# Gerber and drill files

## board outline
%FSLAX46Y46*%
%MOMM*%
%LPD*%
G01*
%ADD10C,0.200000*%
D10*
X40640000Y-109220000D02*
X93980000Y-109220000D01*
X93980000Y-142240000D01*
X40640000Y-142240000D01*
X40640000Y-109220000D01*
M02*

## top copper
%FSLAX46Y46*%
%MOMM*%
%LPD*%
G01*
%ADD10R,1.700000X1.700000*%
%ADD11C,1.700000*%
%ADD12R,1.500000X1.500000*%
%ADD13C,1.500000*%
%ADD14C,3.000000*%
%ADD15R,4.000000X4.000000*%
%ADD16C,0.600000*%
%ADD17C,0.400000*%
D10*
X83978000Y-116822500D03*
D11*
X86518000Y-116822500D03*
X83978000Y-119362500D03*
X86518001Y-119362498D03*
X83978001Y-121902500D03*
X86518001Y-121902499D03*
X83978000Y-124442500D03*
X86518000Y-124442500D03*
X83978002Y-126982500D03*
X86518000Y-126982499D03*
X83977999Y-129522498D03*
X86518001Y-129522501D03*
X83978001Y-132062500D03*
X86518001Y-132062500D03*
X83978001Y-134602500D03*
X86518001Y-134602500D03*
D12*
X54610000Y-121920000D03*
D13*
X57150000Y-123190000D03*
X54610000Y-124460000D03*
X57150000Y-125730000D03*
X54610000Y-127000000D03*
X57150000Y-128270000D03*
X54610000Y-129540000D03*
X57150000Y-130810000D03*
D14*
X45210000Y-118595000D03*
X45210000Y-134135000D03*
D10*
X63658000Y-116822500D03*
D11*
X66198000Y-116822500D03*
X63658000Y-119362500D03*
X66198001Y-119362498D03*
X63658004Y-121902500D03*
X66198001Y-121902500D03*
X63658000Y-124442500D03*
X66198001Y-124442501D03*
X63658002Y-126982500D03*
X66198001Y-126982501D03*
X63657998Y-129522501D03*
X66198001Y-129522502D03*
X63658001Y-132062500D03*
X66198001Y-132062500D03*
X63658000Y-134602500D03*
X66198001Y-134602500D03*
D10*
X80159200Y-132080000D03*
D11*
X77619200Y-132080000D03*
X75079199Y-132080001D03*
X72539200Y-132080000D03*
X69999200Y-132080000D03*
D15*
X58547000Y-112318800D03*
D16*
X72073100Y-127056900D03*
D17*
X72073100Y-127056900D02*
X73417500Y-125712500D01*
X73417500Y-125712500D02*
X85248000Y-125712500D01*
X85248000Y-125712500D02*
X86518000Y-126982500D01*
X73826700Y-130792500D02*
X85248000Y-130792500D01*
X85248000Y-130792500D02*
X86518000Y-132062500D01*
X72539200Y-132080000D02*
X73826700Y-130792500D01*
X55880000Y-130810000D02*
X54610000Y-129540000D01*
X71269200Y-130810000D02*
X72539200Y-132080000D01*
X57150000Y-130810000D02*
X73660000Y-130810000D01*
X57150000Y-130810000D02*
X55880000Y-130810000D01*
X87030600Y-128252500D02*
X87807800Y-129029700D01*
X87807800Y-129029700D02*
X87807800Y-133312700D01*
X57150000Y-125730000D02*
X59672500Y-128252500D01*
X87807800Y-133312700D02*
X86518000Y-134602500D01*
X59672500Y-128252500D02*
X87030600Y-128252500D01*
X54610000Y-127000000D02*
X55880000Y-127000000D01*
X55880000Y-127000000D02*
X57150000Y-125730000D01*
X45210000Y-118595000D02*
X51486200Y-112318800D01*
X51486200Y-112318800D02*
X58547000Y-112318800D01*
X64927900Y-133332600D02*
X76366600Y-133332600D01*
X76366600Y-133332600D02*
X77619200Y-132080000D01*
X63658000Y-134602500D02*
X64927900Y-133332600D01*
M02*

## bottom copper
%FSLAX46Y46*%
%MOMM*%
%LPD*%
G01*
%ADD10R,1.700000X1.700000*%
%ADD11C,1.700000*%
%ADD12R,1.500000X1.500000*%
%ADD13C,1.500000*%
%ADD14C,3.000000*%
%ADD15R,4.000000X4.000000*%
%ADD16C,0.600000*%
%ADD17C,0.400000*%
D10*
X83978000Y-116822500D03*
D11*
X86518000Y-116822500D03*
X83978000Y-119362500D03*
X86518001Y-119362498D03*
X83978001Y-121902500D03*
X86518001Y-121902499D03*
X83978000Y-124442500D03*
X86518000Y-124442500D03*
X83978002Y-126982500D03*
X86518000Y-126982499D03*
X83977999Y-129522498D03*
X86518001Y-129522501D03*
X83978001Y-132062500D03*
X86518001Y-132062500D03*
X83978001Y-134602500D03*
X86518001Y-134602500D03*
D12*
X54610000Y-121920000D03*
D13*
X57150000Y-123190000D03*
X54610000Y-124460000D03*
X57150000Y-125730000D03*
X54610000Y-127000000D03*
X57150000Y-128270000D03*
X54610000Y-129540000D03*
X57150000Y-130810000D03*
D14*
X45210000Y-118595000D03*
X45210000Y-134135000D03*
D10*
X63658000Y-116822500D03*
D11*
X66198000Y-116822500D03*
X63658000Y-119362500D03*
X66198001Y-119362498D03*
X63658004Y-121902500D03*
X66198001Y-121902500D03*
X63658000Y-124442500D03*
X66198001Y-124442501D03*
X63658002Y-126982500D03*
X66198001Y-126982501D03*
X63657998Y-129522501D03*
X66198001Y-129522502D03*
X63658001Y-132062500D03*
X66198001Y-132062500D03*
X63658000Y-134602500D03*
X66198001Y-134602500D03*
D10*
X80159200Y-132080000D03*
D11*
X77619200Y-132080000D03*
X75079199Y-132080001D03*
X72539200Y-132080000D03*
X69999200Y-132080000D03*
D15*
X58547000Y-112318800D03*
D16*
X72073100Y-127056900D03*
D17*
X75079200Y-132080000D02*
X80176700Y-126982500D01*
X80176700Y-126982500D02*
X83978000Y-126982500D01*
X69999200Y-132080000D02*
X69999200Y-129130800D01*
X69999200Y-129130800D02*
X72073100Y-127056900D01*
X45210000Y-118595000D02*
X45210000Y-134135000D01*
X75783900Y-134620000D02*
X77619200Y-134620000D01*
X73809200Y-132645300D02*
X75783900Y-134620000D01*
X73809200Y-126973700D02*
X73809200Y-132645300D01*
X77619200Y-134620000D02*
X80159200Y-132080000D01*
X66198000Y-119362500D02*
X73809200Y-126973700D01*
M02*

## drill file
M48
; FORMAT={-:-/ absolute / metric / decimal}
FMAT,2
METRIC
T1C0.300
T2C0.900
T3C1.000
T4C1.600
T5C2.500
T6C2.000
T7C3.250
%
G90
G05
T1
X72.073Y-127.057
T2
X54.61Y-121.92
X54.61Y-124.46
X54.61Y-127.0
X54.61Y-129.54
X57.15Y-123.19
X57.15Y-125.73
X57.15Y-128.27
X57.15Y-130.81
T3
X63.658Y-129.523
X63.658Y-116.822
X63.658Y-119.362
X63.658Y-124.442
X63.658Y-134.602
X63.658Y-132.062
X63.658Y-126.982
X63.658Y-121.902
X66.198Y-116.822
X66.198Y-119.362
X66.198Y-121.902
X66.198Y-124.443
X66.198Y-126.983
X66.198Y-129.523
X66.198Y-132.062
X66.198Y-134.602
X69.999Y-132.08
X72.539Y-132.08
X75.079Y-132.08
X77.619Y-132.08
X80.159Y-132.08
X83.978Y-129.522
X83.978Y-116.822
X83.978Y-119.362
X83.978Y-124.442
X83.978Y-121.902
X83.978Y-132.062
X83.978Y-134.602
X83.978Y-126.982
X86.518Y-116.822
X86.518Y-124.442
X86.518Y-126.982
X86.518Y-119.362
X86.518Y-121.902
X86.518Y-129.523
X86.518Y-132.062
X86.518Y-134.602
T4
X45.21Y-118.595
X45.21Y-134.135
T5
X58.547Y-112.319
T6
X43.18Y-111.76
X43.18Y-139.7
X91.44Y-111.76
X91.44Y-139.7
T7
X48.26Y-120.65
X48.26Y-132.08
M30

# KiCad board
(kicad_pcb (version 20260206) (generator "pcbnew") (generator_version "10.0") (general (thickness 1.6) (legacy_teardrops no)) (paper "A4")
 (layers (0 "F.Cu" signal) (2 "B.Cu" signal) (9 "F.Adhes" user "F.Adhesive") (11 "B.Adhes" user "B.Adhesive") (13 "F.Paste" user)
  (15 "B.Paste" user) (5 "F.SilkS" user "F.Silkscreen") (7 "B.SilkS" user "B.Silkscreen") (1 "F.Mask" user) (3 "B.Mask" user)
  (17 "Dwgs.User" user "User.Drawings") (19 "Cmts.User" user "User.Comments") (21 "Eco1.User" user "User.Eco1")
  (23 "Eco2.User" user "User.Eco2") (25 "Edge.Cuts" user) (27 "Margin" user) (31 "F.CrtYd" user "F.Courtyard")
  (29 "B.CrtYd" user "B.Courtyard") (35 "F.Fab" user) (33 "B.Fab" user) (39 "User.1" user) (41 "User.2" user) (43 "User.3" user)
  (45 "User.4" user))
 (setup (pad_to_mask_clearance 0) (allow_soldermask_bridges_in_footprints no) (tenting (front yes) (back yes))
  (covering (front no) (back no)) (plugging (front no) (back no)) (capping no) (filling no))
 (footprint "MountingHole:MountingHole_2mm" (layer "F.Cu") (at 43.18 139.7 90)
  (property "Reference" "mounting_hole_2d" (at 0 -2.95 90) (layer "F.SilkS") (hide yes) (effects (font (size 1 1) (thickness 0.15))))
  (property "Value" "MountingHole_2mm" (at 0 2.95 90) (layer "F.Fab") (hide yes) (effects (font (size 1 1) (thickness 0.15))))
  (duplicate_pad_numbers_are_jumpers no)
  (pad "" np_thru_hole circle (at 0 0 90) (size 2 2) (drill 2) (layers "*.Cu" "*.Mask")))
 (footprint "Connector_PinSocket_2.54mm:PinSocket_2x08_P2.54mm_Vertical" (layer "F.Cu") (at 86.5688 116.8225)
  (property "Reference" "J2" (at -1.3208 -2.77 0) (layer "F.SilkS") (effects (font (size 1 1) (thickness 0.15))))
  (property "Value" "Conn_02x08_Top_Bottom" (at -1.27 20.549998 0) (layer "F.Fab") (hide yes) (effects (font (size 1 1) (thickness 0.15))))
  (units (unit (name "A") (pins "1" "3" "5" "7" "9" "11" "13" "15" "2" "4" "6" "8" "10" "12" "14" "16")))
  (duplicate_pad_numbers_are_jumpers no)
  (pad "1" thru_hole rect (at -2.5908 0) (size 1.7 1.7) (drill 1) (layers "*.Cu" "*.Mask") (remove_unused_layers no)
   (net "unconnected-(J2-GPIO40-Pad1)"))
  (pad "2" thru_hole circle (at -0.0508 0) (size 1.7 1.7) (drill 1) (layers "*.Cu" "*.Mask") (remove_unused_layers no)
   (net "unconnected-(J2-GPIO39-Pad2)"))
  (pad "3" thru_hole circle (at -2.5908 2.54) (size 1.7 1.7) (drill 1) (layers "*.Cu" "*.Mask") (remove_unused_layers no)
   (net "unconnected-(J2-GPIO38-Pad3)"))
  (pad "4" thru_hole circle (at -0.050799 2.539998) (size 1.7 1.7) (drill 1) (layers "*.Cu" "*.Mask") (remove_unused_layers no)
   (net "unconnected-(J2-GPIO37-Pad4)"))
  (pad "5" thru_hole circle (at -2.590799 5.08) (size 1.7 1.7) (drill 1) (layers "*.Cu" "*.Mask") (remove_unused_layers no)
   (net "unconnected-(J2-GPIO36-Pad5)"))
  (pad "6" thru_hole circle (at -0.050799 5.079999) (size 1.7 1.7) (drill 1) (layers "*.Cu" "*.Mask") (remove_unused_layers no)
   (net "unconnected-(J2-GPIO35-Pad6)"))
  (pad "7" thru_hole circle (at -2.5908 7.62) (size 1.7 1.7) (drill 1) (layers "*.Cu" "*.Mask") (remove_unused_layers no)
   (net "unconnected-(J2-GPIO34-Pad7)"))
  (pad "8" thru_hole circle (at -0.0508 7.62) (size 1.7 1.7) (drill 1) (layers "*.Cu" "*.Mask") (remove_unused_layers no)
   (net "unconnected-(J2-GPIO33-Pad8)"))
  (pad "9" thru_hole circle (at -2.590798 10.16) (size 1.7 1.7) (drill 1) (layers "*.Cu" "*.Mask") (remove_unused_layers no) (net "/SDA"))
  (pad "10" thru_hole circle (at -0.0508 10.159999) (size 1.7 1.7) (drill 1) (layers "*.Cu" "*.Mask") (remove_unused_layers no) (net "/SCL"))
  (pad "11" thru_hole circle (at -2.590801 12.699998) (size 1.7 1.7) (drill 1) (layers "*.Cu" "*.Mask") (remove_unused_layers no)
   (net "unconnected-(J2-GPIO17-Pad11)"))
  (pad "12" thru_hole circle (at -0.050799 12.700001) (size 1.7 1.7) (drill 1) (layers "*.Cu" "*.Mask") (remove_unused_layers no)
   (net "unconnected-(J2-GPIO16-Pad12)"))
  (pad "13" thru_hole circle (at -2.590799 15.24) (size 1.7 1.7) (drill 1) (layers "*.Cu" "*.Mask") (remove_unused_layers no)
   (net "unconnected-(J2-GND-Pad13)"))
  (pad "14" thru_hole circle (at -0.050799 15.24) (size 1.7 1.7) (drill 1) (layers "*.Cu" "*.Mask") (remove_unused_layers no) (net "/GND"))
  (pad "15" thru_hole circle (at -2.590799 17.78) (size 1.7 1.7) (drill 1) (layers "*.Cu" "*.Mask") (remove_unused_layers no)
   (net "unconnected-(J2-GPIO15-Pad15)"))
  (pad "16" thru_hole circle (at -0.050799 17.78) (size 1.7 1.7) (drill 1) (layers "*.Cu" "*.Mask") (remove_unused_layers no) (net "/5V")))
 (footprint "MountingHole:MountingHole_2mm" (layer "F.Cu") (at 91.44 111.76 90)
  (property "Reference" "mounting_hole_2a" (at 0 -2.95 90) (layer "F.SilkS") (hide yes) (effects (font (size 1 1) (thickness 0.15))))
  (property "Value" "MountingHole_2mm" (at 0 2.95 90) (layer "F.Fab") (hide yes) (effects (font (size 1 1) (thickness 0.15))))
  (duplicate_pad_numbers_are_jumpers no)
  (pad "" np_thru_hole circle (at 0 0 90) (size 2 2) (drill 2) (layers "*.Cu" "*.Mask")))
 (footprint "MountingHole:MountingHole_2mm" (layer "F.Cu") (at 43.18 111.76 90)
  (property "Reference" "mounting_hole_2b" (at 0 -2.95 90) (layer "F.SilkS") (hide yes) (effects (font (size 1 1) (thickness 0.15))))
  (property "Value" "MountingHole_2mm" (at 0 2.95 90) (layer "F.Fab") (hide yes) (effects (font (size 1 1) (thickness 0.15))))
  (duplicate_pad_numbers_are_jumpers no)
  (pad "" np_thru_hole circle (at 0 0 90) (size 2 2) (drill 2) (layers "*.Cu" "*.Mask")))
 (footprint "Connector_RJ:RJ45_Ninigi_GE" (layer "F.Cu") (at 54.61 121.92 -90)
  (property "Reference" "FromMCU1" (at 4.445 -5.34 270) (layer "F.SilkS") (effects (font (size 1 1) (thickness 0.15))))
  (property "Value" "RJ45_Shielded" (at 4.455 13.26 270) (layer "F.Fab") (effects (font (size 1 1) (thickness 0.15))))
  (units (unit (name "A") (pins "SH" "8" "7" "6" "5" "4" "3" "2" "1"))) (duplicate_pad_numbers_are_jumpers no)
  (pad "" np_thru_hole circle (at -1.27 6.35 270) (size 3.25 3.25) (drill 3.25) (layers "*.Cu" "*.Mask"))
  (pad "" np_thru_hole circle (at 10.16 6.35 90) (size 3.25 3.25) (drill 3.25) (layers "*.Cu" "*.Mask"))
  (pad "1" thru_hole rect (at 0 0 90) (size 1.5 1.5) (drill 0.9) (layers "*.Cu" "*.Mask") (remove_unused_layers no)
   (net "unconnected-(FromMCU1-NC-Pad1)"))
  (pad "2" thru_hole circle (at 1.27 -2.54 90) (size 1.5 1.5) (drill 0.9) (layers "*.Cu" "*.Mask") (remove_unused_layers no)
   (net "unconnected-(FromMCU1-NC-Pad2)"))
  (pad "3" thru_hole circle (at 2.54 0 90) (size 1.5 1.5) (drill 0.9) (layers "*.Cu" "*.Mask") (remove_unused_layers no)
   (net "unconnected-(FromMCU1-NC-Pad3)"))
  (pad "4" thru_hole circle (at 3.81 -2.54 90) (size 1.5 1.5) (drill 0.9) (layers "*.Cu" "*.Mask") (remove_unused_layers no) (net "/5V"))
  (pad "5" thru_hole circle (at 5.08 0 90) (size 1.5 1.5) (drill 0.9) (layers "*.Cu" "*.Mask") (remove_unused_layers no) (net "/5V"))
  (pad "6" thru_hole circle (at 6.35 -2.54 90) (size 1.5 1.5) (drill 0.9) (layers "*.Cu" "*.Mask") (remove_unused_layers no)
   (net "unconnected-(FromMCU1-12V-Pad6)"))
  (pad "7" thru_hole circle (at 7.62 0 90) (size 1.5 1.5) (drill 0.9) (layers "*.Cu" "*.Mask") (remove_unused_layers no) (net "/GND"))
  (pad "8" thru_hole circle (at 8.89 -2.54 90) (size 1.5 1.5) (drill 0.9) (layers "*.Cu" "*.Mask") (remove_unused_layers no) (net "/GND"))
  (pad "SH" thru_hole circle (at -3.325 9.4 270) (size 3 3) (drill 1.6) (layers "*.Cu" "*.Mask") (remove_unused_layers no)
   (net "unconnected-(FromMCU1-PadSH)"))
  (pad "SH" thru_hole circle (at 12.215 9.4 90) (size 3 3) (drill 1.6) (layers "*.Cu" "*.Mask") (remove_unused_layers no)
   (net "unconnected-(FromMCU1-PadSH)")))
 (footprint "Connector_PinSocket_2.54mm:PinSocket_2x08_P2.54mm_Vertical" (layer "F.Cu") (at 66.2488 116.8225)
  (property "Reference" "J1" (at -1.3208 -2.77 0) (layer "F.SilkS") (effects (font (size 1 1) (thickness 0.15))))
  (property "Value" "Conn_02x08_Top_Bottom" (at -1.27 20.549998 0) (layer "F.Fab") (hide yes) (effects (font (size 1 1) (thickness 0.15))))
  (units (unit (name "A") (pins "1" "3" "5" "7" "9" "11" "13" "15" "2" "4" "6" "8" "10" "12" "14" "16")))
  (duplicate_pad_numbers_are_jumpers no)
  (pad "1" thru_hole rect (at -2.5908 0) (size 1.7 1.7) (drill 1) (layers "*.Cu" "*.Mask") (remove_unused_layers no)
   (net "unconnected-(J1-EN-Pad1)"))
  (pad "2" thru_hole circle (at -0.0508 0) (size 1.7 1.7) (drill 1) (layers "*.Cu" "*.Mask") (remove_unused_layers no)
   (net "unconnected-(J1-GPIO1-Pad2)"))
  (pad "3" thru_hole circle (at -2.5908 2.54) (size 1.7 1.7) (drill 1) (layers "*.Cu" "*.Mask") (remove_unused_layers no)
   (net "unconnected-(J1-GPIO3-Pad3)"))
  (pad "4" thru_hole circle (at -0.050799 2.539998) (size 1.7 1.7) (drill 1) (layers "*.Cu" "*.Mask") (remove_unused_layers no) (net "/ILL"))
  (pad "5" thru_hole circle (at -2.590796 5.08) (size 1.7 1.7) (drill 1) (layers "*.Cu" "*.Mask") (remove_unused_layers no)
   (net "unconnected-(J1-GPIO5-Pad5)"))
  (pad "6" thru_hole circle (at -0.050799 5.08) (size 1.7 1.7) (drill 1) (layers "*.Cu" "*.Mask") (remove_unused_layers no)
   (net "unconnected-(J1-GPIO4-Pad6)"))
  (pad "7" thru_hole circle (at -2.5908 7.62) (size 1.7 1.7) (drill 1) (layers "*.Cu" "*.Mask") (remove_unused_layers no)
   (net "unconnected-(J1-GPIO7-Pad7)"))
  (pad "8" thru_hole circle (at -0.050799 7.620001) (size 1.7 1.7) (drill 1) (layers "*.Cu" "*.Mask") (remove_unused_layers no)
   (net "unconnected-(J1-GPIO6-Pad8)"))
  (pad "9" thru_hole circle (at -2.590798 10.16) (size 1.7 1.7) (drill 1) (layers "*.Cu" "*.Mask") (remove_unused_layers no)
   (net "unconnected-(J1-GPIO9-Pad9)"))
  (pad "10" thru_hole circle (at -0.050799 10.160001) (size 1.7 1.7) (drill 1) (layers "*.Cu" "*.Mask") (remove_unused_layers no)
   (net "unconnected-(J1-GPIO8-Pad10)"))
  (pad "11" thru_hole circle (at -2.590802 12.700001) (size 1.7 1.7) (drill 1) (layers "*.Cu" "*.Mask") (remove_unused_layers no)
   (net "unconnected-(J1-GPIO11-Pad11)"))
  (pad "12" thru_hole circle (at -0.050799 12.700002) (size 1.7 1.7) (drill 1) (layers "*.Cu" "*.Mask") (remove_unused_layers no)
   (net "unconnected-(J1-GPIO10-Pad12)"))
  (pad "13" thru_hole circle (at -2.590799 15.24) (size 1.7 1.7) (drill 1) (layers "*.Cu" "*.Mask") (remove_unused_layers no)
   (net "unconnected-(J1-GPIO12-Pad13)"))
  (pad "14" thru_hole circle (at -0.050799 15.24) (size 1.7 1.7) (drill 1) (layers "*.Cu" "*.Mask") (remove_unused_layers no)
   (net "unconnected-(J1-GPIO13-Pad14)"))
  (pad "15" thru_hole circle (at -2.5908 17.78) (size 1.7 1.7) (drill 1) (layers "*.Cu" "*.Mask") (remove_unused_layers no) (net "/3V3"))
  (pad "16" thru_hole circle (at -0.050799 17.78) (size 1.7 1.7) (drill 1) (layers "*.Cu" "*.Mask") (remove_unused_layers no)
   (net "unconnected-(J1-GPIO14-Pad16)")))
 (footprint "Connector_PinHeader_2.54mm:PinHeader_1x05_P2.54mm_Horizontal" (layer "F.Cu") (at 80.1592 132.08 -90)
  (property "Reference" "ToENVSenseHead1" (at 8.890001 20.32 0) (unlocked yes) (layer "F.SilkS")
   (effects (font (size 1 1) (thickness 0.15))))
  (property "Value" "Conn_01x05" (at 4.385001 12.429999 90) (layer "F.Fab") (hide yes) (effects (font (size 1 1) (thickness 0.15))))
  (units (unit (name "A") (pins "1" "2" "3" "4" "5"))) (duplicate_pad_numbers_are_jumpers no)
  (pad "1" thru_hole rect (at 0 0 270) (size 1.7 1.7) (drill 1) (layers "*.Cu" "*.Mask") (remove_unused_layers no) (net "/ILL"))
  (pad "2" thru_hole circle (at 0 2.54 270) (size 1.7 1.7) (drill 1) (layers "*.Cu" "*.Mask") (remove_unused_layers no) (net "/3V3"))
  (pad "3" thru_hole circle (at 0.000001 5.080001 270) (size 1.7 1.7) (drill 1) (layers "*.Cu" "*.Mask") (remove_unused_layers no)
   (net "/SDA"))
  (pad "4" thru_hole circle (at 0 7.62 270) (size 1.7 1.7) (drill 1) (layers "*.Cu" "*.Mask") (remove_unused_layers no) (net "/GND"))
  (pad "5" thru_hole circle (at 0 10.16 270) (size 1.7 1.7) (drill 1) (layers "*.Cu" "*.Mask") (remove_unused_layers no) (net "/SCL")))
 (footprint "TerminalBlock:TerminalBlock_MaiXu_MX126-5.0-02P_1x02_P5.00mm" (layer "F.Cu") (at 58.547 112.3188)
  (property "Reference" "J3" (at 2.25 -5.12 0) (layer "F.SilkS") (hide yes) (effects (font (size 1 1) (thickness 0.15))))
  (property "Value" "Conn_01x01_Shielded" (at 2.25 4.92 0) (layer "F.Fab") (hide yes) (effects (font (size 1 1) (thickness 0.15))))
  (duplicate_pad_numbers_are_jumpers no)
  (pad "1" thru_hole rect (at 0 0) (size 4 4) (drill 2.5) (layers "*.Cu" "*.Mask") (remove_unused_layers no)
   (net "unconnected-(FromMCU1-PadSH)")))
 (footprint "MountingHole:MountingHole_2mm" (layer "F.Cu") (at 91.44 139.7 90)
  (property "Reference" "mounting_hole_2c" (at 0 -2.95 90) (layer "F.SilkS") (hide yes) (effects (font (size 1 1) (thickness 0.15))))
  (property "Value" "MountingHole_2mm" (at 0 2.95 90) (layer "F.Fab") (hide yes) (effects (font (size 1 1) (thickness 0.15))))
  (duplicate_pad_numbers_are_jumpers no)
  (pad "" np_thru_hole circle (at 0 0 90) (size 2 2) (drill 2) (layers "*.Cu" "*.Mask")))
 (gr_rect (start 40.64 109.22) (end 93.98 142.24) (stroke (width 0.2) (type solid)) (fill no) (layer "Edge.Cuts"))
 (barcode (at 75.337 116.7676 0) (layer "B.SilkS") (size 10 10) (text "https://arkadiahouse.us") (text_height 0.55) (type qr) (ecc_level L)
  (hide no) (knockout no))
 (segment (start 75.0792 132.08) (end 80.1767 126.9825) (width 0.4) (layer "B.Cu") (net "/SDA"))
 (segment (start 80.1767 126.9825) (end 83.978 126.9825) (width 0.4) (layer "B.Cu") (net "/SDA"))
 (segment (start 72.0731 127.0569) (end 73.4175 125.7125) (width 0.4) (layer "F.Cu") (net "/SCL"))
 (segment (start 73.4175 125.7125) (end 85.248 125.7125) (width 0.4) (layer "F.Cu") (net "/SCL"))
 (segment (start 85.248 125.7125) (end 86.518 126.9825) (width 0.4) (layer "F.Cu") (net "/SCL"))
 (via (at 72.0731 127.0569) (size 0.6) (drill 0.3) (layers "F.Cu" "B.Cu") (capping no) (covering (front no) (back no))
  (plugging (front no) (back no)) (filling no) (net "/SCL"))
 (segment (start 69.9992 132.08) (end 69.9992 129.1308) (width 0.4) (layer "B.Cu") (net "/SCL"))
 (segment (start 69.9992 129.1308) (end 72.0731 127.0569) (width 0.4) (layer "B.Cu") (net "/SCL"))
 (segment (start 73.8267 130.7925) (end 85.248 130.7925) (width 0.4) (layer "F.Cu") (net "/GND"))
 (segment (start 85.248 130.7925) (end 86.518 132.0625) (width 0.4) (layer "F.Cu") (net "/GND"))
 (segment (start 72.5392 132.08) (end 73.8267 130.7925) (width 0.4) (layer "F.Cu") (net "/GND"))
 (segment (start 55.88 130.81) (end 54.61 129.54) (width 0.4) (layer "F.Cu") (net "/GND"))
 (segment (start 71.2692 130.81) (end 72.5392 132.08) (width 0.4) (layer "F.Cu") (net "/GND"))
 (segment (start 57.15 130.81) (end 73.66 130.81) (width 0.4) (layer "F.Cu") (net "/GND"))
 (segment (start 57.15 130.81) (end 55.88 130.81) (width 0.4) (layer "F.Cu") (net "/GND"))
 (segment (start 87.0306 128.2525) (end 87.8078 129.0297) (width 0.4) (layer "F.Cu") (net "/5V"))
 (segment (start 87.8078 129.0297) (end 87.8078 133.3127) (width 0.4) (layer "F.Cu") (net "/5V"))
 (segment (start 57.15 125.73) (end 59.6725 128.2525) (width 0.4) (layer "F.Cu") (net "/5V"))
 (segment (start 87.8078 133.3127) (end 86.518 134.6025) (width 0.4) (layer "F.Cu") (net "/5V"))
 (segment (start 59.6725 128.2525) (end 87.0306 128.2525) (width 0.4) (layer "F.Cu") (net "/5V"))
 (segment (start 54.61 127) (end 55.88 127) (width 0.4) (layer "F.Cu") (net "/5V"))
 (segment (start 55.88 127) (end 57.15 125.73) (width 0.4) (layer "F.Cu") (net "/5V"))
 (segment (start 45.21 118.595) (end 51.4862 112.3188) (width 0.4) (layer "F.Cu") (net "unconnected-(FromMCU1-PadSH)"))
 (segment (start 51.4862 112.3188) (end 58.547 112.3188) (width 0.4) (layer "F.Cu") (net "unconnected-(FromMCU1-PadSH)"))
 (segment (start 45.21 118.595) (end 45.21 134.135) (width 0.4) (layer "B.Cu") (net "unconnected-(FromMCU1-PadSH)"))
 (segment (start 75.7839 134.62) (end 77.6192 134.62) (width 0.4) (layer "B.Cu") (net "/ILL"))
 (segment (start 73.8092 132.6453) (end 75.7839 134.62) (width 0.4) (layer "B.Cu") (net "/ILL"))
 (segment (start 73.8092 126.9737) (end 73.8092 132.6453) (width 0.4) (layer "B.Cu") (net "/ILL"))
 (segment (start 77.6192 134.62) (end 80.1592 132.08) (width 0.4) (layer "B.Cu") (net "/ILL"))
 (segment (start 66.198 119.3625) (end 73.8092 126.9737) (width 0.4) (layer "B.Cu") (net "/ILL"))
 (segment (start 64.9279 133.3326) (end 76.3666 133.3326) (width 0.4) (layer "F.Cu") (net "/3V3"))
 (segment (start 76.3666 133.3326) (end 77.6192 132.08) (width 0.4) (layer "F.Cu") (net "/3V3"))
 (segment (start 63.658 134.6025) (end 64.9279 133.3326) (width 0.4) (layer "F.Cu") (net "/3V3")))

